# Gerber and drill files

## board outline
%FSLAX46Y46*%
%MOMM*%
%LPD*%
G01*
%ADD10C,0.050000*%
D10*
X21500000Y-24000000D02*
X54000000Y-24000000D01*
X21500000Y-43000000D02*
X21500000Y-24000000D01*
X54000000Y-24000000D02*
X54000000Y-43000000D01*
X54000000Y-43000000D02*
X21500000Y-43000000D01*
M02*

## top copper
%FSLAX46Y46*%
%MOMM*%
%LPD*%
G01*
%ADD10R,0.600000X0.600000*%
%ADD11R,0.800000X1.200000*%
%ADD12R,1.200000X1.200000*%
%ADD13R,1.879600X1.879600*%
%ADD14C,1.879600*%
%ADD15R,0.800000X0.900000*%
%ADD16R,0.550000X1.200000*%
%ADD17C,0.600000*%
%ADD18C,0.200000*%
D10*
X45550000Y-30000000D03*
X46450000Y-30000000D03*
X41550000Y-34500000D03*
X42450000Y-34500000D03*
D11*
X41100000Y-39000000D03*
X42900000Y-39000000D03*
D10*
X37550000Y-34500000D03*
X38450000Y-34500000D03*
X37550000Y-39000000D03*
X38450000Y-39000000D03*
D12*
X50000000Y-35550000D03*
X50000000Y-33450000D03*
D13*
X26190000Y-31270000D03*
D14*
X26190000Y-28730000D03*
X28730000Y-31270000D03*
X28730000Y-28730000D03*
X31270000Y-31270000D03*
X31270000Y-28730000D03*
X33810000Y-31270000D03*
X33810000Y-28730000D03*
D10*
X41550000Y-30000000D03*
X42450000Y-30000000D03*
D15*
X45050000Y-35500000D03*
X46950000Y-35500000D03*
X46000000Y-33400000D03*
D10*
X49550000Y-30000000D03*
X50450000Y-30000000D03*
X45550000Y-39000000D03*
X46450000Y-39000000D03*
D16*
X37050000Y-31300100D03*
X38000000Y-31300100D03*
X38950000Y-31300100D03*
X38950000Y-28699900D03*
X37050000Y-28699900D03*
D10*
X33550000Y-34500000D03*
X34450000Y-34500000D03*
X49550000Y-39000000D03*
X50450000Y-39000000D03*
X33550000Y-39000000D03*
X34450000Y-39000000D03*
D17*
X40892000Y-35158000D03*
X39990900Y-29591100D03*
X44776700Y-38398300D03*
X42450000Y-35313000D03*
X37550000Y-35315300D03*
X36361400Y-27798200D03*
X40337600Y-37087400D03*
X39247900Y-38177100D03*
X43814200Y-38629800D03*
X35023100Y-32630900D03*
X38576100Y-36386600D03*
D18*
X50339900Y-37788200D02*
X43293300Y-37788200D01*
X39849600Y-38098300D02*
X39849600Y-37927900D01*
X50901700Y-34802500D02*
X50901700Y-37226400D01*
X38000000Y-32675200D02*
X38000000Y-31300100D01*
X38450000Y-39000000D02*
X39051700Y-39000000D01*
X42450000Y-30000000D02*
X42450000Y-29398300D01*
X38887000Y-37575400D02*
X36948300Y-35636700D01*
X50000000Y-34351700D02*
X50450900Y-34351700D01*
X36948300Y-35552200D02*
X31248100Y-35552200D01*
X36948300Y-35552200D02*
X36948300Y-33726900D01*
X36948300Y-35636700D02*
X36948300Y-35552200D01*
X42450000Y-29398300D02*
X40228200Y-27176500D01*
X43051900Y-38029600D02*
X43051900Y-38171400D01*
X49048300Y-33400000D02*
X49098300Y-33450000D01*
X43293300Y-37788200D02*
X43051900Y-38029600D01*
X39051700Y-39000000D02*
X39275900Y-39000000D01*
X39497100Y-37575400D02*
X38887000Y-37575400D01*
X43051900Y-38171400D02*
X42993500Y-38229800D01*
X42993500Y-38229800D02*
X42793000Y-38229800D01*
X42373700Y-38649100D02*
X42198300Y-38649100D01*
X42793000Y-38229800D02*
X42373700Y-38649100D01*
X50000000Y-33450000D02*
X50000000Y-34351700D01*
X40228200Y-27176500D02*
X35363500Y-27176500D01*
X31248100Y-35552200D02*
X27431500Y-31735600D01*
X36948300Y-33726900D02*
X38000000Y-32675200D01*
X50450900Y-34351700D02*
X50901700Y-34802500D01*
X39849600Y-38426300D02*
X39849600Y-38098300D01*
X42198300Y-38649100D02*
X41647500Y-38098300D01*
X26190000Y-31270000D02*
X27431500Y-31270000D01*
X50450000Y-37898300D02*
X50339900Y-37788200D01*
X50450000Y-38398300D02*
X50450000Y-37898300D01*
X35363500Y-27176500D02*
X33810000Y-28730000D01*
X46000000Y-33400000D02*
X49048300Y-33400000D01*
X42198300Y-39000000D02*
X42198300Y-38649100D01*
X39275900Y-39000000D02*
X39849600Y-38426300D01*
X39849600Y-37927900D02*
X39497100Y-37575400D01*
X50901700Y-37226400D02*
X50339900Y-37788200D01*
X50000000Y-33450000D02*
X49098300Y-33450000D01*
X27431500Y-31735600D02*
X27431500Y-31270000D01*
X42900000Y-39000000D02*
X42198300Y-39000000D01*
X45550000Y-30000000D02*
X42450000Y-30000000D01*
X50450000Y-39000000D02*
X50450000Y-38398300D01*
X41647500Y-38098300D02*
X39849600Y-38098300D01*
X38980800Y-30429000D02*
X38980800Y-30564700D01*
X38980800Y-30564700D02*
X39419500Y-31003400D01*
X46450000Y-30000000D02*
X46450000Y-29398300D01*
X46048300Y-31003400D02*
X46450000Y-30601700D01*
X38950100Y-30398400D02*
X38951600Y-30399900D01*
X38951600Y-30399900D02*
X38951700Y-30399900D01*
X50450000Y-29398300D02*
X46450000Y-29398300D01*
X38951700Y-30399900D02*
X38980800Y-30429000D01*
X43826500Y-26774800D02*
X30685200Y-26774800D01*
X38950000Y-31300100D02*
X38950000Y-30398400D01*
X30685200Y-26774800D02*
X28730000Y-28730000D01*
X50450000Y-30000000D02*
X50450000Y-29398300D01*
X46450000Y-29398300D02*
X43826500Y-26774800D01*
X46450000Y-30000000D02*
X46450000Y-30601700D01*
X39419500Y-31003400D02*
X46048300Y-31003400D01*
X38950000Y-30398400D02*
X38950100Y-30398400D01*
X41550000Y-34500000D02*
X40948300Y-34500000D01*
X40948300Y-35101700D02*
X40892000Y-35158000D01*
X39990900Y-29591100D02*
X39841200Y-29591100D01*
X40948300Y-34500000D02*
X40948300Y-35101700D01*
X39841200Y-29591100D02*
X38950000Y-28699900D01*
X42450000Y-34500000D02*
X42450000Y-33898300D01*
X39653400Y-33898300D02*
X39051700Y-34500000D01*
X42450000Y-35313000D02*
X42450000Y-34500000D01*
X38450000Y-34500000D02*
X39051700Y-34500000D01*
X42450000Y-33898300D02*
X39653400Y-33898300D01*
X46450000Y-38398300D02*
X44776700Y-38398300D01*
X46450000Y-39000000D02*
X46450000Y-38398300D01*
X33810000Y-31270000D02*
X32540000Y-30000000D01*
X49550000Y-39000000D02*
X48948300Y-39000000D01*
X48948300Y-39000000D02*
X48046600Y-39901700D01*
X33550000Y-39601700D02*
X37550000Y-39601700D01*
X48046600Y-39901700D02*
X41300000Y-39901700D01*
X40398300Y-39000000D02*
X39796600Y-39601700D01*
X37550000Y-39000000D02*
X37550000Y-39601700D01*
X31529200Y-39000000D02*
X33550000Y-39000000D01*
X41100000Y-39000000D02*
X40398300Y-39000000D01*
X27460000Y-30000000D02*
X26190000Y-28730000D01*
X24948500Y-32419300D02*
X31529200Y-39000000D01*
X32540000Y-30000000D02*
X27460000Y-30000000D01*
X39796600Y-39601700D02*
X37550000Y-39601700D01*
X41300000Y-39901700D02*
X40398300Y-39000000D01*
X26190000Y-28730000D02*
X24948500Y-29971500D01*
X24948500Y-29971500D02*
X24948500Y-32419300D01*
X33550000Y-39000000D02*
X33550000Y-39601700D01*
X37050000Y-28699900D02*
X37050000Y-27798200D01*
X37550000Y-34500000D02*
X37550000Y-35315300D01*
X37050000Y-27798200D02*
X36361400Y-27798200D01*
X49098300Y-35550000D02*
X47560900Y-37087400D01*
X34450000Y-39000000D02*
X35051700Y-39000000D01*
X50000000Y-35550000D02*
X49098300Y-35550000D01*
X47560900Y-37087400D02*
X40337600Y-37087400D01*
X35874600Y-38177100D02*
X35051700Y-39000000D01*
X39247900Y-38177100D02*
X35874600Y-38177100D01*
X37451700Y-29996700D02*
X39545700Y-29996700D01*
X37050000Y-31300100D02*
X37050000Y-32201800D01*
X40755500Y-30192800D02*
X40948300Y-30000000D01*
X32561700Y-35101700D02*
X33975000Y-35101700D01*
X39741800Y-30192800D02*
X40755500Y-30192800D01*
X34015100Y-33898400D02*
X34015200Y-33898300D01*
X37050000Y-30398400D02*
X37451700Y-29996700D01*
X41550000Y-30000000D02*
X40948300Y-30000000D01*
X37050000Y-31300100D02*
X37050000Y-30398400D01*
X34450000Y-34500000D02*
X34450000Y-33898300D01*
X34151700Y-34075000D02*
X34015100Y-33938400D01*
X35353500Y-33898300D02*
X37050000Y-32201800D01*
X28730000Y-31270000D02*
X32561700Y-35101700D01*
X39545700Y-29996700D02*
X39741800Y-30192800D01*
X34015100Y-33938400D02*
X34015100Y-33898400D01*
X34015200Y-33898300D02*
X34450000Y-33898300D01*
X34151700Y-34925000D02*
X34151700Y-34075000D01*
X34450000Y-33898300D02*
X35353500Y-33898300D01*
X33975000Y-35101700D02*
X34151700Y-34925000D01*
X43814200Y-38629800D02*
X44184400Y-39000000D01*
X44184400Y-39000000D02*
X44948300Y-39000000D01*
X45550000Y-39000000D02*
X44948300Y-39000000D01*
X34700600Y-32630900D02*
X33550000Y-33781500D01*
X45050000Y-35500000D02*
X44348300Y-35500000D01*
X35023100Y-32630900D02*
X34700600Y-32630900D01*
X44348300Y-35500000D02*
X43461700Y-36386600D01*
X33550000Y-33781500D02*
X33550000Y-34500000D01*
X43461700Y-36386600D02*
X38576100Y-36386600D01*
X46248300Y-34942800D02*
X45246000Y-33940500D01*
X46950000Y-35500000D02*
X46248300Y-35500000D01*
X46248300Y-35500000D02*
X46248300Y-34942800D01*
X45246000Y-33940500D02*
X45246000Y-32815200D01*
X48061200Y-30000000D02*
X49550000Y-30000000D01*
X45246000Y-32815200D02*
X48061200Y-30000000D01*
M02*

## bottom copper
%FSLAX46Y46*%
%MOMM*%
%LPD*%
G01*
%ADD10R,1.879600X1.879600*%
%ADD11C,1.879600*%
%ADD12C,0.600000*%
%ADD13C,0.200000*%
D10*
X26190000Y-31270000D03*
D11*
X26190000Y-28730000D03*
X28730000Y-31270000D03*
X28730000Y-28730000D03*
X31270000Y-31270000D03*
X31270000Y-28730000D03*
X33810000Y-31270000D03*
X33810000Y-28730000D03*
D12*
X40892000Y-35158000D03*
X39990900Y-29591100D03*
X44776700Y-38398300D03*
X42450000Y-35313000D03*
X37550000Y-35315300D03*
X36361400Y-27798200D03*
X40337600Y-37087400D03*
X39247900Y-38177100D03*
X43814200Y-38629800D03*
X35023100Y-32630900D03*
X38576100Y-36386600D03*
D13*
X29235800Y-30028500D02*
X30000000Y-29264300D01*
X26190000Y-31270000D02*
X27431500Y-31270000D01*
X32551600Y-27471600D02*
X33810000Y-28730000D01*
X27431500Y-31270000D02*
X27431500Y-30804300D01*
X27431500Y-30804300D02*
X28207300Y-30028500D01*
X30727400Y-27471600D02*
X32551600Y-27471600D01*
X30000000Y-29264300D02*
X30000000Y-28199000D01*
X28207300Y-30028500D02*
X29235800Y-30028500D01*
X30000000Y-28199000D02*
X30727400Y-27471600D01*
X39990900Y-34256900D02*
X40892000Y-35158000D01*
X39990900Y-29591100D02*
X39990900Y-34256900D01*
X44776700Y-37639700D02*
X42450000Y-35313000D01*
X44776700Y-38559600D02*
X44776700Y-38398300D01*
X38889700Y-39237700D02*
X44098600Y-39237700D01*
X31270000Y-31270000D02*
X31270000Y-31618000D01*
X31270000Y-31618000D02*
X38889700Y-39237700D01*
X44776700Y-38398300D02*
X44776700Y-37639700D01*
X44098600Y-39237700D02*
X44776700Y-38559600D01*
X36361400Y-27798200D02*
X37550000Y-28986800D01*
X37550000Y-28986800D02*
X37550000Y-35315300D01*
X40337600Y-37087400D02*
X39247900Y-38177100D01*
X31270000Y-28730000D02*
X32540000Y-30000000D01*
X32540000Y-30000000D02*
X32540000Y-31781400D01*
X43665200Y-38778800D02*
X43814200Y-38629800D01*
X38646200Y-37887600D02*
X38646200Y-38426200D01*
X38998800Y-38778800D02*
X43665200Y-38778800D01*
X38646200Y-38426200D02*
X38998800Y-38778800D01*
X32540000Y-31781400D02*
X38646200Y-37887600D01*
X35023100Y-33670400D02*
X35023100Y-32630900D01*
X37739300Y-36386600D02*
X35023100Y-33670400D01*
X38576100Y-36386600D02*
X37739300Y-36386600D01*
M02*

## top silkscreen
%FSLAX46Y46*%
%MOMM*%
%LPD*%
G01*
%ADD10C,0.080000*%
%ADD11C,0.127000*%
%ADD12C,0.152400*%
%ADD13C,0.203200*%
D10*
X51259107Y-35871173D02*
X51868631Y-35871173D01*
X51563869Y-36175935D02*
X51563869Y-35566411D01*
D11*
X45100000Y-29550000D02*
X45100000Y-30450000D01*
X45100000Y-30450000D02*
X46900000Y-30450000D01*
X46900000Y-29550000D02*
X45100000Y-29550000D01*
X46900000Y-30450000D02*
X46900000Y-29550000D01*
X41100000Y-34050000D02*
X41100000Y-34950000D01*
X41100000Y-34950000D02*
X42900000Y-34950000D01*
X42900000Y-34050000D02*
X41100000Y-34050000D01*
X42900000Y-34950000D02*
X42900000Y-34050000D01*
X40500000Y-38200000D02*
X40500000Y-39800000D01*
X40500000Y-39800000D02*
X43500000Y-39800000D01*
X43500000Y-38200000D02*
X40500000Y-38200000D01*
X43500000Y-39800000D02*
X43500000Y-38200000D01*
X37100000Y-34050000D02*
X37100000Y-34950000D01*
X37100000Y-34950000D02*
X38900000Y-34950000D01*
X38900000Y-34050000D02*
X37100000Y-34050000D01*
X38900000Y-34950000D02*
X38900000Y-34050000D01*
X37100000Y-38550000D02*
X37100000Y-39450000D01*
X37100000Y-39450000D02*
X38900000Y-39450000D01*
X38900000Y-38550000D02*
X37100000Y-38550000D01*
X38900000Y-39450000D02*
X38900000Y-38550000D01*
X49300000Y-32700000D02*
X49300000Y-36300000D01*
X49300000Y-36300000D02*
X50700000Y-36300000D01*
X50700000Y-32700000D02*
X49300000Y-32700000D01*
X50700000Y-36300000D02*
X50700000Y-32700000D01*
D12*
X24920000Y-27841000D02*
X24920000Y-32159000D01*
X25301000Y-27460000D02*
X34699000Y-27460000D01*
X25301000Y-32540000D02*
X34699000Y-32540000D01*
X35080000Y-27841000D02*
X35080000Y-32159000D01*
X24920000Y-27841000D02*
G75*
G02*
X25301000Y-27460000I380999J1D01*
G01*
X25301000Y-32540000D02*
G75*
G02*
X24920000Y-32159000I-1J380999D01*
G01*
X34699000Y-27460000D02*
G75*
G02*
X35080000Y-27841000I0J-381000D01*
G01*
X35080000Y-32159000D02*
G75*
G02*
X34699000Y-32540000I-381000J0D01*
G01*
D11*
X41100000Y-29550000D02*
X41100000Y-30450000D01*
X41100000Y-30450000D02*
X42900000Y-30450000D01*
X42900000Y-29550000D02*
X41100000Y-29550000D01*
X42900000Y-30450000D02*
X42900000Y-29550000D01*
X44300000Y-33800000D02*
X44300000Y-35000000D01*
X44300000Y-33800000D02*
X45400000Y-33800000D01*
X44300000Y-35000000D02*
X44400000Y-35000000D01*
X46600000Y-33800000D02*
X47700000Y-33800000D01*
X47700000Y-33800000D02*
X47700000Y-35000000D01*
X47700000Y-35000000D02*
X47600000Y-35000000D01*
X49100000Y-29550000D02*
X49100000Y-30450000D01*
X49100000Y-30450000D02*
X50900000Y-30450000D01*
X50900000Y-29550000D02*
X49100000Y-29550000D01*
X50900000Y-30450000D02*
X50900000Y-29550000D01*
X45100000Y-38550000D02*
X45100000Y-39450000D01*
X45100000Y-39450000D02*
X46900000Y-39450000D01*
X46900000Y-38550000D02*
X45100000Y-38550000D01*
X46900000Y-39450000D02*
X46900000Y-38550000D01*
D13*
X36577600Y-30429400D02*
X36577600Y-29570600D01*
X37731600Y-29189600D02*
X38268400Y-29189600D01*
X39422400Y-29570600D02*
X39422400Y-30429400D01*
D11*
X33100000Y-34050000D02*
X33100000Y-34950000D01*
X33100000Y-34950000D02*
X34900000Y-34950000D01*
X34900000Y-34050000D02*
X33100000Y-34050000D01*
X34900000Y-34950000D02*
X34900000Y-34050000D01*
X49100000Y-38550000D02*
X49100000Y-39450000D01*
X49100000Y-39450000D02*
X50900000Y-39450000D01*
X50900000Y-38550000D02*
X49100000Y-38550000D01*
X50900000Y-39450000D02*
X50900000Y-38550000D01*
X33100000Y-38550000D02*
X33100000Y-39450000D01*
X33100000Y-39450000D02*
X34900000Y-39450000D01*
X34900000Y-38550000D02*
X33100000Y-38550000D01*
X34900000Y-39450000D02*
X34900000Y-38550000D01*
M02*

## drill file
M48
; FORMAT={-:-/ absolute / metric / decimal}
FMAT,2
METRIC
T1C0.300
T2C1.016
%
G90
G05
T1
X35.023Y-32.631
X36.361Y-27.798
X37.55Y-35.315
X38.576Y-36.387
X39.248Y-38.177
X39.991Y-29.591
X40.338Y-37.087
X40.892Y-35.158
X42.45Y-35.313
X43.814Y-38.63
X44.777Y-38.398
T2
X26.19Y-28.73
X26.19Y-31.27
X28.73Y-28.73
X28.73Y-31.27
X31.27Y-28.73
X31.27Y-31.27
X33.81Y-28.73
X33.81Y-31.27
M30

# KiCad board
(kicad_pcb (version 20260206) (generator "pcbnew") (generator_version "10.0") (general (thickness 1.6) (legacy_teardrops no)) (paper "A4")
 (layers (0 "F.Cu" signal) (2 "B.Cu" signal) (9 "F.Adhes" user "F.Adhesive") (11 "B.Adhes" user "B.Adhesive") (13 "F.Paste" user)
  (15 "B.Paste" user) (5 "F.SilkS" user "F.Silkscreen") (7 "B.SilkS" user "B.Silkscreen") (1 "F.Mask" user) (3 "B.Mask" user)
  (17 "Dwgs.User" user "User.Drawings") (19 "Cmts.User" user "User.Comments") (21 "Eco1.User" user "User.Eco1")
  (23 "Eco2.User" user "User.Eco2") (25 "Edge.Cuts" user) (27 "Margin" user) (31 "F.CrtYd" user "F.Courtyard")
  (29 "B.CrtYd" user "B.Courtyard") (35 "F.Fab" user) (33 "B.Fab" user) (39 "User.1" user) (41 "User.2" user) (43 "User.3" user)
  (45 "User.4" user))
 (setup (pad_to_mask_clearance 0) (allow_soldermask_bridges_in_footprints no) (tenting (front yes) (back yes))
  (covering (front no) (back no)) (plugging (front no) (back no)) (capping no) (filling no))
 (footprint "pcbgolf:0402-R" (layer "F.Cu") (at 46 30)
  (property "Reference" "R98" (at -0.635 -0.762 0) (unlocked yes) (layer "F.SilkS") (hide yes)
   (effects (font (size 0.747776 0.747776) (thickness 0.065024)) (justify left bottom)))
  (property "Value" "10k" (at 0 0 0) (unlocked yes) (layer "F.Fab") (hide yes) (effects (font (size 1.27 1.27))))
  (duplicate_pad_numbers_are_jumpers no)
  (fp_line (start -0.9 -0.45) (end -0.9 0.45) (stroke (width 0.127) (type solid)) (layer "F.SilkS"))
  (fp_line (start -0.9 0.45) (end 0.9 0.45) (stroke (width 0.127) (type solid)) (layer "F.SilkS"))
  (fp_line (start 0.9 -0.45) (end -0.9 -0.45) (stroke (width 0.127) (type solid)) (layer "F.SilkS"))
  (fp_line (start 0.9 0.45) (end 0.9 -0.45) (stroke (width 0.127) (type solid)) (layer "F.SilkS"))
  (pad "1" smd rect (at -0.45 0) (size 0.6 0.6) (layers "F.Cu" "F.Mask" "F.Paste") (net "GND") (solder_mask_margin 0.0508)
   (solder_paste_margin 0) (thermal_bridge_angle 0))
  (pad "2" smd rect (at 0.45 0) (size 0.6 0.6) (layers "F.Cu" "F.Mask" "F.Paste") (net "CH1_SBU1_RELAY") (solder_mask_margin 0.0508)
   (solder_paste_margin 0) (thermal_bridge_angle 0)))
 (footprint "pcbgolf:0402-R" (layer "F.Cu") (at 42 34.5)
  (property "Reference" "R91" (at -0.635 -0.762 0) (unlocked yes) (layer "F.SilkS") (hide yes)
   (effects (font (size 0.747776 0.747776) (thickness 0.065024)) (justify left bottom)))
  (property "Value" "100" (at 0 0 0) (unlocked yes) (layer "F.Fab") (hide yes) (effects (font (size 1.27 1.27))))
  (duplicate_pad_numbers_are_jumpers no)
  (fp_line (start -0.9 -0.45) (end -0.9 0.45) (stroke (width 0.127) (type solid)) (layer "F.SilkS"))
  (fp_line (start -0.9 0.45) (end 0.9 0.45) (stroke (width 0.127) (type solid)) (layer "F.SilkS"))
  (fp_line (start 0.9 -0.45) (end -0.9 -0.45) (stroke (width 0.127) (type solid)) (layer "F.SilkS"))
  (fp_line (start 0.9 0.45) (end 0.9 -0.45) (stroke (width 0.127) (type solid)) (layer "F.SilkS"))
  (pad "1" smd rect (at -0.45 0) (size 0.6 0.6) (layers "F.Cu" "F.Mask" "F.Paste") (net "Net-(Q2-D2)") (solder_mask_margin 0.0508)
   (solder_paste_margin 0) (thermal_bridge_angle 0))
  (pad "2" smd rect (at 0.45 0) (size 0.6 0.6) (layers "F.Cu" "F.Mask" "F.Paste") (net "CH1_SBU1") (solder_mask_margin 0.0508)
   (solder_paste_margin 0) (thermal_bridge_angle 0)))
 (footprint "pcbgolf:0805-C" (layer "F.Cu") (at 42 39)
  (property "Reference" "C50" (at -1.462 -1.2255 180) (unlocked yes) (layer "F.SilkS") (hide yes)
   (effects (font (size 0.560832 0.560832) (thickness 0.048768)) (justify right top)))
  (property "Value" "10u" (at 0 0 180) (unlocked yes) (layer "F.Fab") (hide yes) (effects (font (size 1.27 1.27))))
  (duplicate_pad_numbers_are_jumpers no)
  (fp_line (start -1.5 -0.8) (end -1.5 0.8) (stroke (width 0.127) (type solid)) (layer "F.SilkS"))
  (fp_line (start -1.5 0.8) (end 1.5 0.8) (stroke (width 0.127) (type solid)) (layer "F.SilkS"))
  (fp_line (start 1.5 -0.8) (end -1.5 -0.8) (stroke (width 0.127) (type solid)) (layer "F.SilkS"))
  (fp_line (start 1.5 0.8) (end 1.5 -0.8) (stroke (width 0.127) (type solid)) (layer "F.SilkS"))
  (pad "1" smd rect (at -0.9 0) (size 0.8 1.2) (layers "F.Cu" "F.Mask" "F.Paste") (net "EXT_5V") (solder_mask_margin 0.0508)
   (solder_paste_margin 0) (thermal_bridge_angle 0))
  (pad "2" smd rect (at 0.9 0) (size 0.8 1.2) (layers "F.Cu" "F.Mask" "F.Paste") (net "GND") (solder_mask_margin 0.0508)
   (solder_paste_margin 0) (thermal_bridge_angle 0)))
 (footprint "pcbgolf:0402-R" (layer "F.Cu") (at 38 34.5)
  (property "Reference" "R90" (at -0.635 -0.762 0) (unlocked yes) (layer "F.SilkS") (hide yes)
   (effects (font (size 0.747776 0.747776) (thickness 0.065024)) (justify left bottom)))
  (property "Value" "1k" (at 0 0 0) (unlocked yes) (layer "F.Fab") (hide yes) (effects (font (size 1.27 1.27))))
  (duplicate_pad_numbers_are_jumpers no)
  (fp_line (start -0.9 -0.45) (end -0.9 0.45) (stroke (width 0.127) (type solid)) (layer "F.SilkS"))
  (fp_line (start -0.9 0.45) (end 0.9 0.45) (stroke (width 0.127) (type solid)) (layer "F.SilkS"))
  (fp_line (start 0.9 -0.45) (end -0.9 -0.45) (stroke (width 0.127) (type solid)) (layer "F.SilkS"))
  (fp_line (start 0.9 0.45) (end 0.9 -0.45) (stroke (width 0.127) (type solid)) (layer "F.SilkS"))
  (pad "1" smd rect (at -0.45 0) (size 0.6 0.6) (layers "F.Cu" "F.Mask" "F.Paste") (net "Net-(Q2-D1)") (solder_mask_margin 0.0508)
   (solder_paste_margin 0) (thermal_bridge_angle 0))
  (pad "2" smd rect (at 0.45 0) (size 0.6 0.6) (layers "F.Cu" "F.Mask" "F.Paste") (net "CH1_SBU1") (solder_mask_margin 0.0508)
   (solder_paste_margin 0) (thermal_bridge_angle 0)))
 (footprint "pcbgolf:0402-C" (layer "F.Cu") (at 38 39)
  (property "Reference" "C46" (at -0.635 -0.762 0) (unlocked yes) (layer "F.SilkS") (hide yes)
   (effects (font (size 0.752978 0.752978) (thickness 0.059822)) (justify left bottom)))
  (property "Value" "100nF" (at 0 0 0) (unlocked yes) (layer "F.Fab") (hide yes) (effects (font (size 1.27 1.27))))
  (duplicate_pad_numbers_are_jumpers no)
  (fp_line (start -0.9 -0.45) (end -0.9 0.45) (stroke (width 0.127) (type solid)) (layer "F.SilkS"))
  (fp_line (start -0.9 0.45) (end 0.9 0.45) (stroke (width 0.127) (type solid)) (layer "F.SilkS"))
  (fp_line (start 0.9 -0.45) (end -0.9 -0.45) (stroke (width 0.127) (type solid)) (layer "F.SilkS"))
  (fp_line (start 0.9 0.45) (end 0.9 -0.45) (stroke (width 0.127) (type solid)) (layer "F.SilkS"))
  (pad "1" smd rect (at -0.45 0) (size 0.6 0.6) (layers "F.Cu" "F.Mask" "F.Paste") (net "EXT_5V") (solder_mask_margin 0.0508)
   (solder_paste_margin 0) (thermal_bridge_angle 0))
  (pad "2" smd rect (at 0.45 0) (size 0.6 0.6) (layers "F.Cu" "F.Mask" "F.Paste") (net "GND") (solder_mask_margin 0.0508)
   (solder_paste_margin 0) (thermal_bridge_angle 0)))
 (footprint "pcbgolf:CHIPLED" (layer "F.Cu") (at 50 34.5)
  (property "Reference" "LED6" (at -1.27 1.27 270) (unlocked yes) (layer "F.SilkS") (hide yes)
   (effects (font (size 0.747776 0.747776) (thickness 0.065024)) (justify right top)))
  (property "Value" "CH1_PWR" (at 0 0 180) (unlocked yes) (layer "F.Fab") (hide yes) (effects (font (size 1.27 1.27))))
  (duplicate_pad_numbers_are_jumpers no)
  (fp_line (start -0.7 -1.8) (end -0.7 1.8) (stroke (width 0.127) (type solid)) (layer "F.SilkS"))
  (fp_line (start -0.7 1.8) (end 0.7 1.8) (stroke (width 0.127) (type solid)) (layer "F.SilkS"))
  (fp_line (start 0.7 -1.8) (end -0.7 -1.8) (stroke (width 0.127) (type solid)) (layer "F.SilkS"))
  (fp_line (start 0.7 1.8) (end 0.7 -1.8) (stroke (width 0.127) (type solid)) (layer "F.SilkS"))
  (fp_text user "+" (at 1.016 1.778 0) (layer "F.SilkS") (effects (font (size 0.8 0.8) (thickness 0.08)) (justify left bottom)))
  (pad "A" smd rect (at 0 1.05) (size 1.2 1.2) (layers "F.Cu" "F.Mask" "F.Paste") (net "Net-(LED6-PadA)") (solder_mask_margin 0.0508)
   (solder_paste_margin 0) (thermal_bridge_angle 0))
  (pad "C" smd rect (at 0 -1.05) (size 1.2 1.2) (layers "F.Cu" "F.Mask" "F.Paste") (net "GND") (solder_mask_margin 0.0508)
   (solder_paste_margin 0) (thermal_bridge_angle 0)))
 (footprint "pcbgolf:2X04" (layer "F.Cu") (at 30 30)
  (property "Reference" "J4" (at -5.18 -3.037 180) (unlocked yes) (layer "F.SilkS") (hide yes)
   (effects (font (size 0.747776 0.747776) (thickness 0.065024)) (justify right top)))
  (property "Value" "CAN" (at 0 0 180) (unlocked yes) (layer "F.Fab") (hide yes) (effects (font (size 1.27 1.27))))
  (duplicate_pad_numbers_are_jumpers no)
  (fp_line (start -5.08 -2.159) (end -5.08 2.159) (stroke (width 0.1524) (type solid)) (layer "F.SilkS"))
  (fp_line (start -4.699 -2.54) (end 4.699 -2.54) (stroke (width 0.1524) (type solid)) (layer "F.SilkS"))
  (fp_line (start -4.699 2.54) (end 4.699 2.54) (stroke (width 0.1524) (type solid)) (layer "F.SilkS"))
  (fp_line (start 5.08 -2.159) (end 5.08 2.159) (stroke (width 0.1524) (type solid)) (layer "F.SilkS"))
  (fp_arc (start -5.08 -2.159) (mid -4.968408 -2.428408) (end -4.699 -2.54) (stroke (width 0.1524) (type solid)) (layer "F.SilkS"))
  (fp_arc (start -4.699 2.54) (mid -4.968408 2.428408) (end -5.08 2.159) (stroke (width 0.1524) (type solid)) (layer "F.SilkS"))
  (fp_arc (start 4.699 -2.54) (mid 4.968408 -2.428408) (end 5.08 -2.159) (stroke (width 0.1524) (type solid)) (layer "F.SilkS"))
  (fp_arc (start 5.08 2.159) (mid 4.968408 2.428408) (end 4.699 2.54) (stroke (width 0.1524) (type solid)) (layer "F.SilkS"))
  (pad "1" thru_hole rect (at -3.81 1.27 90) (size 1.8796 1.8796) (drill 1.016) (layers "*.Cu" "*.Mask") (remove_unused_layers no)
   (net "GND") (solder_mask_margin 0.0508) (thermal_bridge_angle 0))
  (pad "2" thru_hole circle (at -3.81 -1.27 90) (size 1.8796 1.8796) (drill 1.016) (layers "*.Cu" "*.Mask") (remove_unused_layers no)
   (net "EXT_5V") (solder_mask_margin 0.0508) (thermal_bridge_angle 0))
  (pad "3" thru_hole circle (at -1.27 1.27 90) (size 1.8796 1.8796) (drill 1.016) (layers "*.Cu" "*.Mask") (remove_unused_layers no)
   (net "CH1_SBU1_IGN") (solder_mask_margin 0.0508) (thermal_bridge_angle 0))
  (pad "4" thru_hole circle (at -1.27 -1.27 90) (size 1.8796 1.8796) (drill 1.016) (layers "*.Cu" "*.Mask") (remove_unused_layers no)
   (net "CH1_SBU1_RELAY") (solder_mask_margin 0.0508) (thermal_bridge_angle 0))
  (pad "5" thru_hole circle (at 1.27 1.27 90) (size 1.8796 1.8796) (drill 1.016) (layers "*.Cu" "*.Mask") (remove_unused_layers no)
   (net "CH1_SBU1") (solder_mask_margin 0.0508) (thermal_bridge_angle 0))
  (pad "6" thru_hole circle (at 1.27 -1.27 90) (size 1.8796 1.8796) (drill 1.016) (layers "*.Cu" "*.Mask") (remove_unused_layers no)
   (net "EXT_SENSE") (solder_mask_margin 0.0508) (thermal_bridge_angle 0))
  (pad "7" thru_hole circle (at 3.81 1.27 90) (size 1.8796 1.8796) (drill 1.016) (layers "*.Cu" "*.Mask") (remove_unused_layers no)
   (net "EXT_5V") (solder_mask_margin 0.0508) (thermal_bridge_angle 0))
  (pad "8" thru_hole circle (at 3.81 -1.27 90) (size 1.8796 1.8796) (drill 1.016) (layers "*.Cu" "*.Mask") (remove_unused_layers no)
   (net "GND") (solder_mask_margin 0.0508) (thermal_bridge_angle 0)))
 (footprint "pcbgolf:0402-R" (layer "F.Cu") (at 42 30)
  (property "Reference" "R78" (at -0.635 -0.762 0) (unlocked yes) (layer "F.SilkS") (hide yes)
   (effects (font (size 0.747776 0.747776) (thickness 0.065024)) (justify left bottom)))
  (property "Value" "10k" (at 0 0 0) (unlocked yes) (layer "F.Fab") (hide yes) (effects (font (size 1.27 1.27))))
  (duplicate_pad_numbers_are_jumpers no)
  (fp_line (start -0.9 -0.45) (end -0.9 0.45) (stroke (width 0.127) (type solid)) (layer "F.SilkS"))
  (fp_line (start -0.9 0.45) (end 0.9 0.45) (stroke (width 0.127) (type solid)) (layer "F.SilkS"))
  (fp_line (start 0.9 -0.45) (end -0.9 -0.45) (stroke (width 0.127) (type solid)) (layer "F.SilkS"))
  (fp_line (start 0.9 0.45) (end 0.9 -0.45) (stroke (width 0.127) (type solid)) (layer "F.SilkS"))
  (pad "1" smd rect (at -0.45 0) (size 0.6 0.6) (layers "F.Cu" "F.Mask" "F.Paste") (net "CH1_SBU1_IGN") (solder_mask_margin 0.0508)
   (solder_paste_margin 0) (thermal_bridge_angle 0))
  (pad "2" smd rect (at 0.45 0) (size 0.6 0.6) (layers "F.Cu" "F.Mask" "F.Paste") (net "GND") (solder_mask_margin 0.0508)
   (solder_paste_margin 0) (thermal_bridge_angle 0)))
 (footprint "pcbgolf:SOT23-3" (layer "F.Cu") (at 46 34.5)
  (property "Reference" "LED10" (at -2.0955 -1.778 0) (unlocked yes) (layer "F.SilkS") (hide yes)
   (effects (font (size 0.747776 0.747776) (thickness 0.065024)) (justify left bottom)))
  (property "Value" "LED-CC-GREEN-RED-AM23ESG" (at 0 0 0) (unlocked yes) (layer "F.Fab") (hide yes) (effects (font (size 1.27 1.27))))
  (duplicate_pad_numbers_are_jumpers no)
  (fp_line (start -1.7 -0.7) (end -1.7 0.5) (stroke (width 0.127) (type solid)) (layer "F.SilkS"))
  (fp_line (start -1.7 -0.7) (end -0.6 -0.7) (stroke (width 0.127) (type solid)) (layer "F.SilkS"))
  (fp_line (start -1.7 0.5) (end -1.6 0.5) (stroke (width 0.127) (type solid)) (layer "F.SilkS"))
  (fp_line (start 0.6 -0.7) (end 1.7 -0.7) (stroke (width 0.127) (type solid)) (layer "F.SilkS"))
  (fp_line (start 1.7 -0.7) (end 1.7 0.5) (stroke (width 0.127) (type solid)) (layer "F.SilkS"))
  (fp_line (start 1.7 0.5) (end 1.6 0.5) (stroke (width 0.127) (type solid)) (layer "F.SilkS"))
  (pad "1" smd rect (at -0.95 1) (size 0.8 0.9) (layers "F.Cu" "F.Mask" "F.Paste") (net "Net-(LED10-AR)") (solder_mask_margin 0.0508)
   (solder_paste_margin 0) (thermal_bridge_angle 0))
  (pad "2" smd rect (at 0.95 1) (size 0.8 0.9) (layers "F.Cu" "F.Mask" "F.Paste") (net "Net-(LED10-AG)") (solder_mask_margin 0.0508)
   (solder_paste_margin 0) (thermal_bridge_angle 0))
  (pad "3" smd rect (at 0 -1.1) (size 0.8 0.9) (layers "F.Cu" "F.Mask" "F.Paste") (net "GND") (solder_mask_margin 0.0508)
   (solder_paste_margin 0) (thermal_bridge_angle 0)))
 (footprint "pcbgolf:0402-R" (layer "F.Cu") (at 50 30)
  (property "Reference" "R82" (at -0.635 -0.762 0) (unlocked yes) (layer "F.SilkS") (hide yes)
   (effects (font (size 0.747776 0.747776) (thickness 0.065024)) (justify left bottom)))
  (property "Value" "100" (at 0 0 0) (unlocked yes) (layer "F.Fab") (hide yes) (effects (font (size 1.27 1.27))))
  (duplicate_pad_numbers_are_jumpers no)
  (fp_line (start -0.9 -0.45) (end -0.9 0.45) (stroke (width 0.127) (type solid)) (layer "F.SilkS"))
  (fp_line (start -0.9 0.45) (end 0.9 0.45) (stroke (width 0.127) (type solid)) (layer "F.SilkS"))
  (fp_line (start 0.9 -0.45) (end -0.9 -0.45) (stroke (width 0.127) (type solid)) (layer "F.SilkS"))
  (fp_line (start 0.9 0.45) (end 0.9 -0.45) (stroke (width 0.127) (type solid)) (layer "F.SilkS"))
  (pad "1" smd rect (at -0.45 0) (size 0.6 0.6) (layers "F.Cu" "F.Mask" "F.Paste") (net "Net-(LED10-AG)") (solder_mask_margin 0.0508)
   (solder_paste_margin 0) (thermal_bridge_angle 0))
  (pad "2" smd rect (at 0.45 0) (size 0.6 0.6) (layers "F.Cu" "F.Mask" "F.Paste") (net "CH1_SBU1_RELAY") (solder_mask_margin 0.0508)
   (solder_paste_margin 0) (thermal_bridge_angle 0)))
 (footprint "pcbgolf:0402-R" (layer "F.Cu") (at 46 39)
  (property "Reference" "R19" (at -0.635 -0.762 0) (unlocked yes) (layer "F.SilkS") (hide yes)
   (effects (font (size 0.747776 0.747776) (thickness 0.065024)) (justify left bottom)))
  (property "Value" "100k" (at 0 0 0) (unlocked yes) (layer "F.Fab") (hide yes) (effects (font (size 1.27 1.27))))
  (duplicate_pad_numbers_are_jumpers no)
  (fp_line (start -0.9 -0.45) (end -0.9 0.45) (stroke (width 0.127) (type solid)) (layer "F.SilkS"))
  (fp_line (start -0.9 0.45) (end 0.9 0.45) (stroke (width 0.127) (type solid)) (layer "F.SilkS"))
  (fp_line (start 0.9 -0.45) (end -0.9 -0.45) (stroke (width 0.127) (type solid)) (layer "F.SilkS"))
  (fp_line (start 0.9 0.45) (end 0.9 -0.45) (stroke (width 0.127) (type solid)) (layer "F.SilkS"))
  (pad "1" smd rect (at -0.45 0) (size 0.6 0.6) (layers "F.Cu" "F.Mask" "F.Paste") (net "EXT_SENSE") (solder_mask_margin 0.0508)
   (solder_paste_margin 0) (thermal_bridge_angle 0))
  (pad "2" smd rect (at 0.45 0) (size 0.6 0.6) (layers "F.Cu" "F.Mask" "F.Paste") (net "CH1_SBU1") (solder_mask_margin 0.0508)
   (solder_paste_margin 0) (thermal_bridge_angle 0)))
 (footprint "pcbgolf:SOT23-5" (layer "F.Cu") (at 38 30)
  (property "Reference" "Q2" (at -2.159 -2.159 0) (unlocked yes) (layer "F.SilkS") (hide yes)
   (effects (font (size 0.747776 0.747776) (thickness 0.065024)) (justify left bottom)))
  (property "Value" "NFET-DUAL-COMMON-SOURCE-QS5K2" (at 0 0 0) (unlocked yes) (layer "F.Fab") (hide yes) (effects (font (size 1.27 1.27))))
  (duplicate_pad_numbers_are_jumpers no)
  (fp_line (start -1.4224 0.4294) (end -1.4224 -0.4294) (stroke (width 0.2032) (type solid)) (layer "F.SilkS"))
  (fp_line (start -0.2684 -0.8104) (end 0.2684 -0.8104) (stroke (width 0.2032) (type solid)) (layer "F.SilkS"))
  (fp_line (start 1.4224 -0.4294) (end 1.4224 0.4294) (stroke (width 0.2032) (type solid)) (layer "F.SilkS"))
  (pad "1" smd rect (at -0.95 1.3001) (size 0.55 1.2) (layers "F.Cu" "F.Mask" "F.Paste") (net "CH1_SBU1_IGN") (solder_mask_margin 0.0508)
   (solder_paste_margin 0) (thermal_bridge_angle 0))
  (pad "2" smd rect (at 0 1.3001) (size 0.55 1.2) (layers "F.Cu" "F.Mask" "F.Paste") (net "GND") (solder_mask_margin 0.0508)
   (solder_paste_margin 0) (thermal_bridge_angle 0))
  (pad "3" smd rect (at 0.95 1.3001) (size 0.55 1.2) (layers "F.Cu" "F.Mask" "F.Paste") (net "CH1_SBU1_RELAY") (solder_mask_margin 0.0508)
   (solder_paste_margin 0) (thermal_bridge_angle 0))
  (pad "4" smd rect (at 0.95 -1.3001) (size 0.55 1.2) (layers "F.Cu" "F.Mask" "F.Paste") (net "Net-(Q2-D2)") (solder_mask_margin 0.0508)
   (solder_paste_margin 0) (thermal_bridge_angle 0))
  (pad "5" smd rect (at -0.95 -1.3001) (size 0.55 1.2) (layers "F.Cu" "F.Mask" "F.Paste") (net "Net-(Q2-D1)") (solder_mask_margin 0.0508)
   (solder_paste_margin 0) (thermal_bridge_angle 0)))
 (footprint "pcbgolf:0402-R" (layer "F.Cu") (at 34 34.5)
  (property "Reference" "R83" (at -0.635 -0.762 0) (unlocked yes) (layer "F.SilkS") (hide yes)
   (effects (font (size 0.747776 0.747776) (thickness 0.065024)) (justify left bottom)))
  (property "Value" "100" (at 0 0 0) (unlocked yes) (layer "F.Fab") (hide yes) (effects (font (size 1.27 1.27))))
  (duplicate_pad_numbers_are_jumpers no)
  (fp_line (start -0.9 -0.45) (end -0.9 0.45) (stroke (width 0.127) (type solid)) (layer "F.SilkS"))
  (fp_line (start -0.9 0.45) (end 0.9 0.45) (stroke (width 0.127) (type solid)) (layer "F.SilkS"))
  (fp_line (start 0.9 -0.45) (end -0.9 -0.45) (stroke (width 0.127) (type solid)) (layer "F.SilkS"))
  (fp_line (start 0.9 0.45) (end 0.9 -0.45) (stroke (width 0.127) (type solid)) (layer "F.SilkS"))
  (pad "1" smd rect (at -0.45 0) (size 0.6 0.6) (layers "F.Cu" "F.Mask" "F.Paste") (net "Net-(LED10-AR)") (solder_mask_margin 0.0508)
   (solder_paste_margin 0) (thermal_bridge_angle 0))
  (pad "2" smd rect (at 0.45 0) (size 0.6 0.6) (layers "F.Cu" "F.Mask" "F.Paste") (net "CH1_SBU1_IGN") (solder_mask_margin 0.0508)
   (solder_paste_margin 0) (thermal_bridge_angle 0)))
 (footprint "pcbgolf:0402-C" (layer "F.Cu") (at 50 39)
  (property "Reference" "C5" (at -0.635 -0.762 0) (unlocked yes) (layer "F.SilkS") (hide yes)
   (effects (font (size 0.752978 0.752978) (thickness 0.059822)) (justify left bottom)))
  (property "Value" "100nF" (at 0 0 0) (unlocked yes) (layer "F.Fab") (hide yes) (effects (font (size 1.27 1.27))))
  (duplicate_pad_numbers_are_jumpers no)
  (fp_line (start -0.9 -0.45) (end -0.9 0.45) (stroke (width 0.127) (type solid)) (layer "F.SilkS"))
  (fp_line (start -0.9 0.45) (end 0.9 0.45) (stroke (width 0.127) (type solid)) (layer "F.SilkS"))
  (fp_line (start 0.9 -0.45) (end -0.9 -0.45) (stroke (width 0.127) (type solid)) (layer "F.SilkS"))
  (fp_line (start 0.9 0.45) (end 0.9 -0.45) (stroke (width 0.127) (type solid)) (layer "F.SilkS"))
  (pad "1" smd rect (at -0.45 0) (size 0.6 0.6) (layers "F.Cu" "F.Mask" "F.Paste") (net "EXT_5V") (solder_mask_margin 0.0508)
   (solder_paste_margin 0) (thermal_bridge_angle 0))
  (pad "2" smd rect (at 0.45 0) (size 0.6 0.6) (layers "F.Cu" "F.Mask" "F.Paste") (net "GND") (solder_mask_margin 0.0508)
   (solder_paste_margin 0) (thermal_bridge_angle 0)))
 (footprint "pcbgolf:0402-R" (layer "F.Cu") (at 34 39)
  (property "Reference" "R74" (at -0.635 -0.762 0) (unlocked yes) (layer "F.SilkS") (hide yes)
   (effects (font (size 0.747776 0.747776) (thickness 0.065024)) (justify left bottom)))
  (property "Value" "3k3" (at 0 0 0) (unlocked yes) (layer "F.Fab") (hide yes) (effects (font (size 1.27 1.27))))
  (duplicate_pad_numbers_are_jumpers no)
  (fp_line (start -0.9 -0.45) (end -0.9 0.45) (stroke (width 0.127) (type solid)) (layer "F.SilkS"))
  (fp_line (start -0.9 0.45) (end 0.9 0.45) (stroke (width 0.127) (type solid)) (layer "F.SilkS"))
  (fp_line (start 0.9 -0.45) (end -0.9 -0.45) (stroke (width 0.127) (type solid)) (layer "F.SilkS"))
  (fp_line (start 0.9 0.45) (end 0.9 -0.45) (stroke (width 0.127) (type solid)) (layer "F.SilkS"))
  (pad "1" smd rect (at -0.45 0) (size 0.6 0.6) (layers "F.Cu" "F.Mask" "F.Paste") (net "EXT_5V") (solder_mask_margin 0.0508)
   (solder_paste_margin 0) (thermal_bridge_angle 0))
  (pad "2" smd rect (at 0.45 0) (size 0.6 0.6) (layers "F.Cu" "F.Mask" "F.Paste") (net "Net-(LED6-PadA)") (solder_mask_margin 0.0508)
   (solder_paste_margin 0) (thermal_bridge_angle 0)))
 (gr_line (start 21.5 24) (end 54 24) (stroke (width 0.05) (type default)) (layer "Edge.Cuts"))
 (gr_line (start 21.5 43) (end 21.5 24) (stroke (width 0.05) (type default)) (layer "Edge.Cuts"))
 (gr_line (start 54 24) (end 54 43) (stroke (width 0.05) (type default)) (layer "Edge.Cuts"))
 (gr_line (start 54 43) (end 21.5 43) (stroke (width 0.05) (type default)) (layer "Edge.Cuts"))
 (segment (start 50.3399 37.7882) (end 43.2933 37.7882) (width 0.2) (layer "F.Cu") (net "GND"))
 (segment (start 39.8496 38.0983) (end 39.8496 37.9279) (width 0.2) (layer "F.Cu") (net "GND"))
 (segment (start 50.9017 34.8025) (end 50.9017 37.2264) (width 0.2) (layer "F.Cu") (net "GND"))
 (segment (start 38 32.6752) (end 38 31.3001) (width 0.2) (layer "F.Cu") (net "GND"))
 (segment (start 38.45 39) (end 39.0517 39) (width 0.2) (layer "F.Cu") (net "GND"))
 (segment (start 42.45 30) (end 42.45 29.3983) (width 0.2) (layer "F.Cu") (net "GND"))
 (segment (start 38.887 37.5754) (end 36.9483 35.6367) (width 0.2) (layer "F.Cu") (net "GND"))
 (segment (start 50 34.3517) (end 50.4509 34.3517) (width 0.2) (layer "F.Cu") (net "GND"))
 (segment (start 36.9483 35.5522) (end 31.2481 35.5522) (width 0.2) (layer "F.Cu") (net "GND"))
 (segment (start 36.9483 35.5522) (end 36.9483 33.7269) (width 0.2) (layer "F.Cu") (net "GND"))
 (segment (start 36.9483 35.6367) (end 36.9483 35.5522) (width 0.2) (layer "F.Cu") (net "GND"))
 (segment (start 42.45 29.3983) (end 40.2282 27.1765) (width 0.2) (layer "F.Cu") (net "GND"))
 (segment (start 43.0519 38.0296) (end 43.0519 38.1714) (width 0.2) (layer "F.Cu") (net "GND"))
 (segment (start 49.0483 33.4) (end 49.0983 33.45) (width 0.2) (layer "F.Cu") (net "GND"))
 (segment (start 43.2933 37.7882) (end 43.0519 38.0296) (width 0.2) (layer "F.Cu") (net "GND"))
 (segment (start 39.0517 39) (end 39.2759 39) (width 0.2) (layer "F.Cu") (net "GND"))
 (segment (start 39.4971 37.5754) (end 38.887 37.5754) (width 0.2) (layer "F.Cu") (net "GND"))
 (segment (start 43.0519 38.1714) (end 42.9935 38.2298) (width 0.2) (layer "F.Cu") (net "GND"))
 (segment (start 42.9935 38.2298) (end 42.793 38.2298) (width 0.2) (layer "F.Cu") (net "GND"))
 (segment (start 42.3737 38.6491) (end 42.1983 38.6491) (width 0.2) (layer "F.Cu") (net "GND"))
 (segment (start 42.793 38.2298) (end 42.3737 38.6491) (width 0.2) (layer "F.Cu") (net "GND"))
 (segment (start 50 33.45) (end 50 34.3517) (width 0.2) (layer "F.Cu") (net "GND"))
 (segment (start 40.2282 27.1765) (end 35.3635 27.1765) (width 0.2) (layer "F.Cu") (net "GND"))
 (segment (start 31.2481 35.5522) (end 27.4315 31.7356) (width 0.2) (layer "F.Cu") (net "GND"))
 (segment (start 36.9483 33.7269) (end 38 32.6752) (width 0.2) (layer "F.Cu") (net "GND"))
 (segment (start 50.4509 34.3517) (end 50.9017 34.8025) (width 0.2) (layer "F.Cu") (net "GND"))
 (segment (start 39.8496 38.4263) (end 39.8496 38.0983) (width 0.2) (layer "F.Cu") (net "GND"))
 (segment (start 42.1983 38.6491) (end 41.6475 38.0983) (width 0.2) (layer "F.Cu") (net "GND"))
 (segment (start 26.19 31.27) (end 27.4315 31.27) (width 0.2) (layer "F.Cu") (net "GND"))
 (segment (start 50.45 37.8983) (end 50.3399 37.7882) (width 0.2) (layer "F.Cu") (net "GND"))
 (segment (start 50.45 38.3983) (end 50.45 37.8983) (width 0.2) (layer "F.Cu") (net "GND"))
 (segment (start 35.3635 27.1765) (end 33.81 28.73) (width 0.2) (layer "F.Cu") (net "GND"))
 (segment (start 46 33.4) (end 49.0483 33.4) (width 0.2) (layer "F.Cu") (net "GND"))
 (segment (start 42.1983 39) (end 42.1983 38.6491) (width 0.2) (layer "F.Cu") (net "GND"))
 (segment (start 39.2759 39) (end 39.8496 38.4263) (width 0.2) (layer "F.Cu") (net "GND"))
 (segment (start 39.8496 37.9279) (end 39.4971 37.5754) (width 0.2) (layer "F.Cu") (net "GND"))
 (segment (start 50.9017 37.2264) (end 50.3399 37.7882) (width 0.2) (layer "F.Cu") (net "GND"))
 (segment (start 50 33.45) (end 49.0983 33.45) (width 0.2) (layer "F.Cu") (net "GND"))
 (segment (start 27.4315 31.7356) (end 27.4315 31.27) (width 0.2) (layer "F.Cu") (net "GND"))
 (segment (start 42.9 39) (end 42.1983 39) (width 0.2) (layer "F.Cu") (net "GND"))
 (segment (start 45.55 30) (end 42.45 30) (width 0.2) (layer "F.Cu") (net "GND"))
 (segment (start 50.45 39) (end 50.45 38.3983) (width 0.2) (layer "F.Cu") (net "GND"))
 (segment (start 41.6475 38.0983) (end 39.8496 38.0983) (width 0.2) (layer "F.Cu") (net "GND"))
 (segment (start 29.2358 30.0285) (end 30 29.2643) (width 0.2) (layer "B.Cu") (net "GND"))
 (segment (start 26.19 31.27) (end 27.4315 31.27) (width 0.2) (layer "B.Cu") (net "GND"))
 (segment (start 32.5516 27.4716) (end 33.81 28.73) (width 0.2) (layer "B.Cu") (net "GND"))
 (segment (start 27.4315 31.27) (end 27.4315 30.8043) (width 0.2) (layer "B.Cu") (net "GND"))
 (segment (start 27.4315 30.8043) (end 28.2073 30.0285) (width 0.2) (layer "B.Cu") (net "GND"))
 (segment (start 30.7274 27.4716) (end 32.5516 27.4716) (width 0.2) (layer "B.Cu") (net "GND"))
 (segment (start 30 29.2643) (end 30 28.199) (width 0.2) (layer "B.Cu") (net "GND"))
 (segment (start 28.2073 30.0285) (end 29.2358 30.0285) (width 0.2) (layer "B.Cu") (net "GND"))
 (segment (start 30 28.199) (end 30.7274 27.4716) (width 0.2) (layer "B.Cu") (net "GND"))
 (segment (start 38.9808 30.429) (end 38.9808 30.5647) (width 0.2) (layer "F.Cu") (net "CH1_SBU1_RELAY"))
 (segment (start 38.9808 30.5647) (end 39.4195 31.0034) (width 0.2) (layer "F.Cu") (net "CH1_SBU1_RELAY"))
 (segment (start 46.45 30) (end 46.45 29.3983) (width 0.2) (layer "F.Cu") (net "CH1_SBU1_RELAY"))
 (segment (start 46.0483 31.0034) (end 46.45 30.6017) (width 0.2) (layer "F.Cu") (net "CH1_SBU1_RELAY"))
 (segment (start 38.9501 30.3984) (end 38.9516 30.3999) (width 0.2) (layer "F.Cu") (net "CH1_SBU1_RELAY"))
 (segment (start 38.9516 30.3999) (end 38.9517 30.3999) (width 0.2) (layer "F.Cu") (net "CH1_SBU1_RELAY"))
 (segment (start 50.45 29.3983) (end 46.45 29.3983) (width 0.2) (layer "F.Cu") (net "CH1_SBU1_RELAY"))
 (segment (start 38.9517 30.3999) (end 38.9808 30.429) (width 0.2) (layer "F.Cu") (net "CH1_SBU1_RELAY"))
 (segment (start 43.8265 26.7748) (end 30.6852 26.7748) (width 0.2) (layer "F.Cu") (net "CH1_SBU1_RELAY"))
 (segment (start 38.95 31.3001) (end 38.95 30.3984) (width 0.2) (layer "F.Cu") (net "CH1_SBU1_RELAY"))
 (segment (start 30.6852 26.7748) (end 28.73 28.73) (width 0.2) (layer "F.Cu") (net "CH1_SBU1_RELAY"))
 (segment (start 50.45 30) (end 50.45 29.3983) (width 0.2) (layer "F.Cu") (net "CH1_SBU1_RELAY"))
 (segment (start 46.45 29.3983) (end 43.8265 26.7748) (width 0.2) (layer "F.Cu") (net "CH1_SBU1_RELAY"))
 (segment (start 46.45 30) (end 46.45 30.6017) (width 0.2) (layer "F.Cu") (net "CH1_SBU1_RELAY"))
 (segment (start 39.4195 31.0034) (end 46.0483 31.0034) (width 0.2) (layer "F.Cu") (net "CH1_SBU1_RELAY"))
 (segment (start 38.95 30.3984) (end 38.9501 30.3984) (width 0.2) (layer "F.Cu") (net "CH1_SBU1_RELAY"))
 (segment (start 41.55 34.5) (end 40.9483 34.5) (width 0.2) (layer "F.Cu") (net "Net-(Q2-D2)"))
 (segment (start 40.9483 35.1017) (end 40.892 35.158) (width 0.2) (layer "F.Cu") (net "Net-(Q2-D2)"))
 (segment (start 39.9909 29.5911) (end 39.8412 29.5911) (width 0.2) (layer "F.Cu") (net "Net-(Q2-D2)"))
 (segment (start 40.9483 34.5) (end 40.9483 35.1017) (width 0.2) (layer "F.Cu") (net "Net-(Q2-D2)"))
 (segment (start 39.8412 29.5911) (end 38.95 28.6999) (width 0.2) (layer "F.Cu") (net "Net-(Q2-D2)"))
 (via (at 40.892 35.158) (size 0.6) (drill 0.3) (layers "F.Cu" "B.Cu") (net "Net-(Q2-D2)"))
 (via (at 39.9909 29.5911) (size 0.6) (drill 0.3) (layers "F.Cu" "B.Cu") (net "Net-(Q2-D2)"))
 (segment (start 39.9909 34.2569) (end 40.892 35.158) (width 0.2) (layer "B.Cu") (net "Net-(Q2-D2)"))
 (segment (start 39.9909 29.5911) (end 39.9909 34.2569) (width 0.2) (layer "B.Cu") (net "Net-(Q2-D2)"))
 (segment (start 42.45 34.5) (end 42.45 33.8983) (width 0.2) (layer "F.Cu") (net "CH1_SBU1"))
 (segment (start 39.6534 33.8983) (end 39.0517 34.5) (width 0.2) (layer "F.Cu") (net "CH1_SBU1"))
 (segment (start 42.45 35.313) (end 42.45 34.5) (width 0.2) (layer "F.Cu") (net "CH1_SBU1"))
 (segment (start 38.45 34.5) (end 39.0517 34.5) (width 0.2) (layer "F.Cu") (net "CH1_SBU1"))
 (segment (start 42.45 33.8983) (end 39.6534 33.8983) (width 0.2) (layer "F.Cu") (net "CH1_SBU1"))
 (segment (start 46.45 38.3983) (end 44.7767 38.3983) (width 0.2) (layer "F.Cu") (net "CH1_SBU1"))
 (segment (start 46.45 39) (end 46.45 38.3983) (width 0.2) (layer "F.Cu") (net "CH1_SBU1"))
 (via (at 44.7767 38.3983) (size 0.6) (drill 0.3) (layers "F.Cu" "B.Cu") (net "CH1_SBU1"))
 (via (at 42.45 35.313) (size 0.6) (drill 0.3) (layers "F.Cu" "B.Cu") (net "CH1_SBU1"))
 (segment (start 44.7767 37.6397) (end 42.45 35.313) (width 0.2) (layer "B.Cu") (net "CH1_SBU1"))
 (segment (start 44.7767 38.5596) (end 44.7767 38.3983) (width 0.2) (layer "B.Cu") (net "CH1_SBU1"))
 (segment (start 38.8897 39.2377) (end 44.0986 39.2377) (width 0.2) (layer "B.Cu") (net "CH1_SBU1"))
 (segment (start 31.27 31.27) (end 31.27 31.618) (width 0.2) (layer "B.Cu") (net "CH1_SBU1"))
 (segment (start 31.27 31.618) (end 38.8897 39.2377) (width 0.2) (layer "B.Cu") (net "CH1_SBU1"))
 (segment (start 44.7767 38.3983) (end 44.7767 37.6397) (width 0.2) (layer "B.Cu") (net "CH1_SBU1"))
 (segment (start 44.0986 39.2377) (end 44.7767 38.5596) (width 0.2) (layer "B.Cu") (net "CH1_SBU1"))
 (segment (start 33.81 31.27) (end 32.54 30) (width 0.2) (layer "F.Cu") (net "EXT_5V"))
 (segment (start 49.55 39) (end 48.9483 39) (width 0.2) (layer "F.Cu") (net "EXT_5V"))
 (segment (start 48.9483 39) (end 48.0466 39.9017) (width 0.2) (layer "F.Cu") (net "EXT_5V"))
 (segment (start 33.55 39.6017) (end 37.55 39.6017) (width 0.2) (layer "F.Cu") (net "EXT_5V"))
 (segment (start 48.0466 39.9017) (end 41.3 39.9017) (width 0.2) (layer "F.Cu") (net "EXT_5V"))
 (segment (start 40.3983 39) (end 39.7966 39.6017) (width 0.2) (layer "F.Cu") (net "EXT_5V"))
 (segment (start 37.55 39) (end 37.55 39.6017) (width 0.2) (layer "F.Cu") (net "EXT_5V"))
 (segment (start 31.5292 39) (end 33.55 39) (width 0.2) (layer "F.Cu") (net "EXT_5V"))
 (segment (start 41.1 39) (end 40.3983 39) (width 0.2) (layer "F.Cu") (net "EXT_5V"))
 (segment (start 27.46 30) (end 26.19 28.73) (width 0.2) (layer "F.Cu") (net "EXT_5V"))
 (segment (start 24.9485 32.4193) (end 31.5292 39) (width 0.2) (layer "F.Cu") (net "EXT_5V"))
 (segment (start 32.54 30) (end 27.46 30) (width 0.2) (layer "F.Cu") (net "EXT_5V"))
 (segment (start 39.7966 39.6017) (end 37.55 39.6017) (width 0.2) (layer "F.Cu") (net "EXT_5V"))
 (segment (start 41.3 39.9017) (end 40.3983 39) (width 0.2) (layer "F.Cu") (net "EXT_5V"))
 (segment (start 26.19 28.73) (end 24.9485 29.9715) (width 0.2) (layer "F.Cu") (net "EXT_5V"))
 (segment (start 24.9485 29.9715) (end 24.9485 32.4193) (width 0.2) (layer "F.Cu") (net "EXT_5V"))
 (segment (start 33.55 39) (end 33.55 39.6017) (width 0.2) (layer "F.Cu") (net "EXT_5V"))
 (segment (start 37.05 28.6999) (end 37.05 27.7982) (width 0.2) (layer "F.Cu") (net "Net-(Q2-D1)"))
 (segment (start 37.55 34.5) (end 37.55 35.3153) (width 0.2) (layer "F.Cu") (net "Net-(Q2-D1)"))
 (segment (start 37.05 27.7982) (end 36.3614 27.7982) (width 0.2) (layer "F.Cu") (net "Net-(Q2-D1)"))
 (via (at 37.55 35.3153) (size 0.6) (drill 0.3) (layers "F.Cu" "B.Cu") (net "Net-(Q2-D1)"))
 (via (at 36.3614 27.7982) (size 0.6) (drill 0.3) (layers "F.Cu" "B.Cu") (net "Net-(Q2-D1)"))
 (segment (start 36.3614 27.7982) (end 37.55 28.9868) (width 0.2) (layer "B.Cu") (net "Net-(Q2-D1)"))
 (segment (start 37.55 28.9868) (end 37.55 35.3153) (width 0.2) (layer "B.Cu") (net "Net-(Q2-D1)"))
 (segment (start 49.0983 35.55) (end 47.5609 37.0874) (width 0.2) (layer "F.Cu") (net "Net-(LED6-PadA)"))
 (segment (start 34.45 39) (end 35.0517 39) (width 0.2) (layer "F.Cu") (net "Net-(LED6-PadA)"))
 (segment (start 50 35.55) (end 49.0983 35.55) (width 0.2) (layer "F.Cu") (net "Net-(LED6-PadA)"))
 (segment (start 47.5609 37.0874) (end 40.3376 37.0874) (width 0.2) (layer "F.Cu") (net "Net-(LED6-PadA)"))
 (segment (start 35.8746 38.1771) (end 35.0517 39) (width 0.2) (layer "F.Cu") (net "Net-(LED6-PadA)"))
 (segment (start 39.2479 38.1771) (end 35.8746 38.1771) (width 0.2) (layer "F.Cu") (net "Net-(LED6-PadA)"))
 (via (at 40.3376 37.0874) (size 0.6) (drill 0.3) (layers "F.Cu" "B.Cu") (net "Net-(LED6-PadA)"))
 (via (at 39.2479 38.1771) (size 0.6) (drill 0.3) (layers "F.Cu" "B.Cu") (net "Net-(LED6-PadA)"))
 (segment (start 40.3376 37.0874) (end 39.2479 38.1771) (width 0.2) (layer "B.Cu") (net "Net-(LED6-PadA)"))
 (segment (start 37.4517 29.9967) (end 39.5457 29.9967) (width 0.2) (layer "F.Cu") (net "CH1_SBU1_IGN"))
 (segment (start 37.05 31.3001) (end 37.05 32.2018) (width 0.2) (layer "F.Cu") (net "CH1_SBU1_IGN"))
 (segment (start 40.7555 30.1928) (end 40.9483 30) (width 0.2) (layer "F.Cu") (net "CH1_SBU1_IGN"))
 (segment (start 32.5617 35.1017) (end 33.975 35.1017) (width 0.2) (layer "F.Cu") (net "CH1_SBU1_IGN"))
 (segment (start 39.7418 30.1928) (end 40.7555 30.1928) (width 0.2) (layer "F.Cu") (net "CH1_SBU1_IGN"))
 (segment (start 34.0151 33.8984) (end 34.0152 33.8983) (width 0.2) (layer "F.Cu") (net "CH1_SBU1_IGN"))
 (segment (start 37.05 30.3984) (end 37.4517 29.9967) (width 0.2) (layer "F.Cu") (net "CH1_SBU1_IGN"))
 (segment (start 41.55 30) (end 40.9483 30) (width 0.2) (layer "F.Cu") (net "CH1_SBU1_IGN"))
 (segment (start 37.05 31.3001) (end 37.05 30.3984) (width 0.2) (layer "F.Cu") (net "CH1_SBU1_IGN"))
 (segment (start 34.45 34.5) (end 34.45 33.8983) (width 0.2) (layer "F.Cu") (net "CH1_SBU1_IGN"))
 (segment (start 34.1517 34.075) (end 34.0151 33.9384) (width 0.2) (layer "F.Cu") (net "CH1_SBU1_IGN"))
 (segment (start 35.3535 33.8983) (end 37.05 32.2018) (width 0.2) (layer "F.Cu") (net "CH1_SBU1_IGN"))
 (segment (start 28.73 31.27) (end 32.5617 35.1017) (width 0.2) (layer "F.Cu") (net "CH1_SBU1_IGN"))
 (segment (start 39.5457 29.9967) (end 39.7418 30.1928) (width 0.2) (layer "F.Cu") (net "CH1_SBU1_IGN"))
 (segment (start 34.0151 33.9384) (end 34.0151 33.8984) (width 0.2) (layer "F.Cu") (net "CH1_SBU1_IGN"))
 (segment (start 34.0152 33.8983) (end 34.45 33.8983) (width 0.2) (layer "F.Cu") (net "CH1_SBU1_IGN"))
 (segment (start 34.1517 34.925) (end 34.1517 34.075) (width 0.2) (layer "F.Cu") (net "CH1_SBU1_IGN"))
 (segment (start 34.45 33.8983) (end 35.3535 33.8983) (width 0.2) (layer "F.Cu") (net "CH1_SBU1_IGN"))
 (segment (start 33.975 35.1017) (end 34.1517 34.925) (width 0.2) (layer "F.Cu") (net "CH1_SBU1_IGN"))
 (segment (start 43.8142 38.6298) (end 44.1844 39) (width 0.2) (layer "F.Cu") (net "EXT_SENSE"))
 (segment (start 44.1844 39) (end 44.9483 39) (width 0.2) (layer "F.Cu") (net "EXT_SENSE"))
 (segment (start 45.55 39) (end 44.9483 39) (width 0.2) (layer "F.Cu") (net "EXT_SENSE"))
 (via (at 43.8142 38.6298) (size 0.6) (drill 0.3) (layers "F.Cu" "B.Cu") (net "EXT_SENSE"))
 (segment (start 31.27 28.73) (end 32.54 30) (width 0.2) (layer "B.Cu") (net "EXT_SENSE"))
 (segment (start 32.54 30) (end 32.54 31.7814) (width 0.2) (layer "B.Cu") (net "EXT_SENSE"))
 (segment (start 43.6652 38.7788) (end 43.8142 38.6298) (width 0.2) (layer "B.Cu") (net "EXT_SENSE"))
 (segment (start 38.6462 37.8876) (end 38.6462 38.4262) (width 0.2) (layer "B.Cu") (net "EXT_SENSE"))
 (segment (start 38.9988 38.7788) (end 43.6652 38.7788) (width 0.2) (layer "B.Cu") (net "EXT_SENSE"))
 (segment (start 38.6462 38.4262) (end 38.9988 38.7788) (width 0.2) (layer "B.Cu") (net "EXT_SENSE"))
 (segment (start 32.54 31.7814) (end 38.6462 37.8876) (width 0.2) (layer "B.Cu") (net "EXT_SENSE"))
 (segment (start 34.7006 32.6309) (end 33.55 33.7815) (width 0.2) (layer "F.Cu") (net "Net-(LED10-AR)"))
 (segment (start 45.05 35.5) (end 44.3483 35.5) (width 0.2) (layer "F.Cu") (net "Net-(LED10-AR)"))
 (segment (start 35.0231 32.6309) (end 34.7006 32.6309) (width 0.2) (layer "F.Cu") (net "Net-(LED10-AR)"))
 (segment (start 44.3483 35.5) (end 43.4617 36.3866) (width 0.2) (layer "F.Cu") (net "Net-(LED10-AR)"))
 (segment (start 33.55 33.7815) (end 33.55 34.5) (width 0.2) (layer "F.Cu") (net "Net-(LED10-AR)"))
 (segment (start 43.4617 36.3866) (end 38.5761 36.3866) (width 0.2) (layer "F.Cu") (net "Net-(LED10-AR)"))
 (via (at 35.0231 32.6309) (size 0.6) (drill 0.3) (layers "F.Cu" "B.Cu") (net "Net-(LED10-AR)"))
 (via (at 38.5761 36.3866) (size 0.6) (drill 0.3) (layers "F.Cu" "B.Cu") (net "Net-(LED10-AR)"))
 (segment (start 35.0231 33.6704) (end 35.0231 32.6309) (width 0.2) (layer "B.Cu") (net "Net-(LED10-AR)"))
 (segment (start 37.7393 36.3866) (end 35.0231 33.6704) (width 0.2) (layer "B.Cu") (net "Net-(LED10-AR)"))
 (segment (start 38.5761 36.3866) (end 37.7393 36.3866) (width 0.2) (layer "B.Cu") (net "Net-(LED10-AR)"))
 (segment (start 46.2483 34.9428) (end 45.246 33.9405) (width 0.2) (layer "F.Cu") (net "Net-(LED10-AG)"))
 (segment (start 46.95 35.5) (end 46.2483 35.5) (width 0.2) (layer "F.Cu") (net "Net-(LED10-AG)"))
 (segment (start 46.2483 35.5) (end 46.2483 34.9428) (width 0.2) (layer "F.Cu") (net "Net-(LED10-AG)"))
 (segment (start 45.246 33.9405) (end 45.246 32.8152) (width 0.2) (layer "F.Cu") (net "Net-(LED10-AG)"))
 (segment (start 48.0612 30) (end 49.55 30) (width 0.2) (layer "F.Cu") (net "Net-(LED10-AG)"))
 (segment (start 45.246 32.8152) (end 48.0612 30) (width 0.2) (layer "F.Cu") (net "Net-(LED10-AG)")))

